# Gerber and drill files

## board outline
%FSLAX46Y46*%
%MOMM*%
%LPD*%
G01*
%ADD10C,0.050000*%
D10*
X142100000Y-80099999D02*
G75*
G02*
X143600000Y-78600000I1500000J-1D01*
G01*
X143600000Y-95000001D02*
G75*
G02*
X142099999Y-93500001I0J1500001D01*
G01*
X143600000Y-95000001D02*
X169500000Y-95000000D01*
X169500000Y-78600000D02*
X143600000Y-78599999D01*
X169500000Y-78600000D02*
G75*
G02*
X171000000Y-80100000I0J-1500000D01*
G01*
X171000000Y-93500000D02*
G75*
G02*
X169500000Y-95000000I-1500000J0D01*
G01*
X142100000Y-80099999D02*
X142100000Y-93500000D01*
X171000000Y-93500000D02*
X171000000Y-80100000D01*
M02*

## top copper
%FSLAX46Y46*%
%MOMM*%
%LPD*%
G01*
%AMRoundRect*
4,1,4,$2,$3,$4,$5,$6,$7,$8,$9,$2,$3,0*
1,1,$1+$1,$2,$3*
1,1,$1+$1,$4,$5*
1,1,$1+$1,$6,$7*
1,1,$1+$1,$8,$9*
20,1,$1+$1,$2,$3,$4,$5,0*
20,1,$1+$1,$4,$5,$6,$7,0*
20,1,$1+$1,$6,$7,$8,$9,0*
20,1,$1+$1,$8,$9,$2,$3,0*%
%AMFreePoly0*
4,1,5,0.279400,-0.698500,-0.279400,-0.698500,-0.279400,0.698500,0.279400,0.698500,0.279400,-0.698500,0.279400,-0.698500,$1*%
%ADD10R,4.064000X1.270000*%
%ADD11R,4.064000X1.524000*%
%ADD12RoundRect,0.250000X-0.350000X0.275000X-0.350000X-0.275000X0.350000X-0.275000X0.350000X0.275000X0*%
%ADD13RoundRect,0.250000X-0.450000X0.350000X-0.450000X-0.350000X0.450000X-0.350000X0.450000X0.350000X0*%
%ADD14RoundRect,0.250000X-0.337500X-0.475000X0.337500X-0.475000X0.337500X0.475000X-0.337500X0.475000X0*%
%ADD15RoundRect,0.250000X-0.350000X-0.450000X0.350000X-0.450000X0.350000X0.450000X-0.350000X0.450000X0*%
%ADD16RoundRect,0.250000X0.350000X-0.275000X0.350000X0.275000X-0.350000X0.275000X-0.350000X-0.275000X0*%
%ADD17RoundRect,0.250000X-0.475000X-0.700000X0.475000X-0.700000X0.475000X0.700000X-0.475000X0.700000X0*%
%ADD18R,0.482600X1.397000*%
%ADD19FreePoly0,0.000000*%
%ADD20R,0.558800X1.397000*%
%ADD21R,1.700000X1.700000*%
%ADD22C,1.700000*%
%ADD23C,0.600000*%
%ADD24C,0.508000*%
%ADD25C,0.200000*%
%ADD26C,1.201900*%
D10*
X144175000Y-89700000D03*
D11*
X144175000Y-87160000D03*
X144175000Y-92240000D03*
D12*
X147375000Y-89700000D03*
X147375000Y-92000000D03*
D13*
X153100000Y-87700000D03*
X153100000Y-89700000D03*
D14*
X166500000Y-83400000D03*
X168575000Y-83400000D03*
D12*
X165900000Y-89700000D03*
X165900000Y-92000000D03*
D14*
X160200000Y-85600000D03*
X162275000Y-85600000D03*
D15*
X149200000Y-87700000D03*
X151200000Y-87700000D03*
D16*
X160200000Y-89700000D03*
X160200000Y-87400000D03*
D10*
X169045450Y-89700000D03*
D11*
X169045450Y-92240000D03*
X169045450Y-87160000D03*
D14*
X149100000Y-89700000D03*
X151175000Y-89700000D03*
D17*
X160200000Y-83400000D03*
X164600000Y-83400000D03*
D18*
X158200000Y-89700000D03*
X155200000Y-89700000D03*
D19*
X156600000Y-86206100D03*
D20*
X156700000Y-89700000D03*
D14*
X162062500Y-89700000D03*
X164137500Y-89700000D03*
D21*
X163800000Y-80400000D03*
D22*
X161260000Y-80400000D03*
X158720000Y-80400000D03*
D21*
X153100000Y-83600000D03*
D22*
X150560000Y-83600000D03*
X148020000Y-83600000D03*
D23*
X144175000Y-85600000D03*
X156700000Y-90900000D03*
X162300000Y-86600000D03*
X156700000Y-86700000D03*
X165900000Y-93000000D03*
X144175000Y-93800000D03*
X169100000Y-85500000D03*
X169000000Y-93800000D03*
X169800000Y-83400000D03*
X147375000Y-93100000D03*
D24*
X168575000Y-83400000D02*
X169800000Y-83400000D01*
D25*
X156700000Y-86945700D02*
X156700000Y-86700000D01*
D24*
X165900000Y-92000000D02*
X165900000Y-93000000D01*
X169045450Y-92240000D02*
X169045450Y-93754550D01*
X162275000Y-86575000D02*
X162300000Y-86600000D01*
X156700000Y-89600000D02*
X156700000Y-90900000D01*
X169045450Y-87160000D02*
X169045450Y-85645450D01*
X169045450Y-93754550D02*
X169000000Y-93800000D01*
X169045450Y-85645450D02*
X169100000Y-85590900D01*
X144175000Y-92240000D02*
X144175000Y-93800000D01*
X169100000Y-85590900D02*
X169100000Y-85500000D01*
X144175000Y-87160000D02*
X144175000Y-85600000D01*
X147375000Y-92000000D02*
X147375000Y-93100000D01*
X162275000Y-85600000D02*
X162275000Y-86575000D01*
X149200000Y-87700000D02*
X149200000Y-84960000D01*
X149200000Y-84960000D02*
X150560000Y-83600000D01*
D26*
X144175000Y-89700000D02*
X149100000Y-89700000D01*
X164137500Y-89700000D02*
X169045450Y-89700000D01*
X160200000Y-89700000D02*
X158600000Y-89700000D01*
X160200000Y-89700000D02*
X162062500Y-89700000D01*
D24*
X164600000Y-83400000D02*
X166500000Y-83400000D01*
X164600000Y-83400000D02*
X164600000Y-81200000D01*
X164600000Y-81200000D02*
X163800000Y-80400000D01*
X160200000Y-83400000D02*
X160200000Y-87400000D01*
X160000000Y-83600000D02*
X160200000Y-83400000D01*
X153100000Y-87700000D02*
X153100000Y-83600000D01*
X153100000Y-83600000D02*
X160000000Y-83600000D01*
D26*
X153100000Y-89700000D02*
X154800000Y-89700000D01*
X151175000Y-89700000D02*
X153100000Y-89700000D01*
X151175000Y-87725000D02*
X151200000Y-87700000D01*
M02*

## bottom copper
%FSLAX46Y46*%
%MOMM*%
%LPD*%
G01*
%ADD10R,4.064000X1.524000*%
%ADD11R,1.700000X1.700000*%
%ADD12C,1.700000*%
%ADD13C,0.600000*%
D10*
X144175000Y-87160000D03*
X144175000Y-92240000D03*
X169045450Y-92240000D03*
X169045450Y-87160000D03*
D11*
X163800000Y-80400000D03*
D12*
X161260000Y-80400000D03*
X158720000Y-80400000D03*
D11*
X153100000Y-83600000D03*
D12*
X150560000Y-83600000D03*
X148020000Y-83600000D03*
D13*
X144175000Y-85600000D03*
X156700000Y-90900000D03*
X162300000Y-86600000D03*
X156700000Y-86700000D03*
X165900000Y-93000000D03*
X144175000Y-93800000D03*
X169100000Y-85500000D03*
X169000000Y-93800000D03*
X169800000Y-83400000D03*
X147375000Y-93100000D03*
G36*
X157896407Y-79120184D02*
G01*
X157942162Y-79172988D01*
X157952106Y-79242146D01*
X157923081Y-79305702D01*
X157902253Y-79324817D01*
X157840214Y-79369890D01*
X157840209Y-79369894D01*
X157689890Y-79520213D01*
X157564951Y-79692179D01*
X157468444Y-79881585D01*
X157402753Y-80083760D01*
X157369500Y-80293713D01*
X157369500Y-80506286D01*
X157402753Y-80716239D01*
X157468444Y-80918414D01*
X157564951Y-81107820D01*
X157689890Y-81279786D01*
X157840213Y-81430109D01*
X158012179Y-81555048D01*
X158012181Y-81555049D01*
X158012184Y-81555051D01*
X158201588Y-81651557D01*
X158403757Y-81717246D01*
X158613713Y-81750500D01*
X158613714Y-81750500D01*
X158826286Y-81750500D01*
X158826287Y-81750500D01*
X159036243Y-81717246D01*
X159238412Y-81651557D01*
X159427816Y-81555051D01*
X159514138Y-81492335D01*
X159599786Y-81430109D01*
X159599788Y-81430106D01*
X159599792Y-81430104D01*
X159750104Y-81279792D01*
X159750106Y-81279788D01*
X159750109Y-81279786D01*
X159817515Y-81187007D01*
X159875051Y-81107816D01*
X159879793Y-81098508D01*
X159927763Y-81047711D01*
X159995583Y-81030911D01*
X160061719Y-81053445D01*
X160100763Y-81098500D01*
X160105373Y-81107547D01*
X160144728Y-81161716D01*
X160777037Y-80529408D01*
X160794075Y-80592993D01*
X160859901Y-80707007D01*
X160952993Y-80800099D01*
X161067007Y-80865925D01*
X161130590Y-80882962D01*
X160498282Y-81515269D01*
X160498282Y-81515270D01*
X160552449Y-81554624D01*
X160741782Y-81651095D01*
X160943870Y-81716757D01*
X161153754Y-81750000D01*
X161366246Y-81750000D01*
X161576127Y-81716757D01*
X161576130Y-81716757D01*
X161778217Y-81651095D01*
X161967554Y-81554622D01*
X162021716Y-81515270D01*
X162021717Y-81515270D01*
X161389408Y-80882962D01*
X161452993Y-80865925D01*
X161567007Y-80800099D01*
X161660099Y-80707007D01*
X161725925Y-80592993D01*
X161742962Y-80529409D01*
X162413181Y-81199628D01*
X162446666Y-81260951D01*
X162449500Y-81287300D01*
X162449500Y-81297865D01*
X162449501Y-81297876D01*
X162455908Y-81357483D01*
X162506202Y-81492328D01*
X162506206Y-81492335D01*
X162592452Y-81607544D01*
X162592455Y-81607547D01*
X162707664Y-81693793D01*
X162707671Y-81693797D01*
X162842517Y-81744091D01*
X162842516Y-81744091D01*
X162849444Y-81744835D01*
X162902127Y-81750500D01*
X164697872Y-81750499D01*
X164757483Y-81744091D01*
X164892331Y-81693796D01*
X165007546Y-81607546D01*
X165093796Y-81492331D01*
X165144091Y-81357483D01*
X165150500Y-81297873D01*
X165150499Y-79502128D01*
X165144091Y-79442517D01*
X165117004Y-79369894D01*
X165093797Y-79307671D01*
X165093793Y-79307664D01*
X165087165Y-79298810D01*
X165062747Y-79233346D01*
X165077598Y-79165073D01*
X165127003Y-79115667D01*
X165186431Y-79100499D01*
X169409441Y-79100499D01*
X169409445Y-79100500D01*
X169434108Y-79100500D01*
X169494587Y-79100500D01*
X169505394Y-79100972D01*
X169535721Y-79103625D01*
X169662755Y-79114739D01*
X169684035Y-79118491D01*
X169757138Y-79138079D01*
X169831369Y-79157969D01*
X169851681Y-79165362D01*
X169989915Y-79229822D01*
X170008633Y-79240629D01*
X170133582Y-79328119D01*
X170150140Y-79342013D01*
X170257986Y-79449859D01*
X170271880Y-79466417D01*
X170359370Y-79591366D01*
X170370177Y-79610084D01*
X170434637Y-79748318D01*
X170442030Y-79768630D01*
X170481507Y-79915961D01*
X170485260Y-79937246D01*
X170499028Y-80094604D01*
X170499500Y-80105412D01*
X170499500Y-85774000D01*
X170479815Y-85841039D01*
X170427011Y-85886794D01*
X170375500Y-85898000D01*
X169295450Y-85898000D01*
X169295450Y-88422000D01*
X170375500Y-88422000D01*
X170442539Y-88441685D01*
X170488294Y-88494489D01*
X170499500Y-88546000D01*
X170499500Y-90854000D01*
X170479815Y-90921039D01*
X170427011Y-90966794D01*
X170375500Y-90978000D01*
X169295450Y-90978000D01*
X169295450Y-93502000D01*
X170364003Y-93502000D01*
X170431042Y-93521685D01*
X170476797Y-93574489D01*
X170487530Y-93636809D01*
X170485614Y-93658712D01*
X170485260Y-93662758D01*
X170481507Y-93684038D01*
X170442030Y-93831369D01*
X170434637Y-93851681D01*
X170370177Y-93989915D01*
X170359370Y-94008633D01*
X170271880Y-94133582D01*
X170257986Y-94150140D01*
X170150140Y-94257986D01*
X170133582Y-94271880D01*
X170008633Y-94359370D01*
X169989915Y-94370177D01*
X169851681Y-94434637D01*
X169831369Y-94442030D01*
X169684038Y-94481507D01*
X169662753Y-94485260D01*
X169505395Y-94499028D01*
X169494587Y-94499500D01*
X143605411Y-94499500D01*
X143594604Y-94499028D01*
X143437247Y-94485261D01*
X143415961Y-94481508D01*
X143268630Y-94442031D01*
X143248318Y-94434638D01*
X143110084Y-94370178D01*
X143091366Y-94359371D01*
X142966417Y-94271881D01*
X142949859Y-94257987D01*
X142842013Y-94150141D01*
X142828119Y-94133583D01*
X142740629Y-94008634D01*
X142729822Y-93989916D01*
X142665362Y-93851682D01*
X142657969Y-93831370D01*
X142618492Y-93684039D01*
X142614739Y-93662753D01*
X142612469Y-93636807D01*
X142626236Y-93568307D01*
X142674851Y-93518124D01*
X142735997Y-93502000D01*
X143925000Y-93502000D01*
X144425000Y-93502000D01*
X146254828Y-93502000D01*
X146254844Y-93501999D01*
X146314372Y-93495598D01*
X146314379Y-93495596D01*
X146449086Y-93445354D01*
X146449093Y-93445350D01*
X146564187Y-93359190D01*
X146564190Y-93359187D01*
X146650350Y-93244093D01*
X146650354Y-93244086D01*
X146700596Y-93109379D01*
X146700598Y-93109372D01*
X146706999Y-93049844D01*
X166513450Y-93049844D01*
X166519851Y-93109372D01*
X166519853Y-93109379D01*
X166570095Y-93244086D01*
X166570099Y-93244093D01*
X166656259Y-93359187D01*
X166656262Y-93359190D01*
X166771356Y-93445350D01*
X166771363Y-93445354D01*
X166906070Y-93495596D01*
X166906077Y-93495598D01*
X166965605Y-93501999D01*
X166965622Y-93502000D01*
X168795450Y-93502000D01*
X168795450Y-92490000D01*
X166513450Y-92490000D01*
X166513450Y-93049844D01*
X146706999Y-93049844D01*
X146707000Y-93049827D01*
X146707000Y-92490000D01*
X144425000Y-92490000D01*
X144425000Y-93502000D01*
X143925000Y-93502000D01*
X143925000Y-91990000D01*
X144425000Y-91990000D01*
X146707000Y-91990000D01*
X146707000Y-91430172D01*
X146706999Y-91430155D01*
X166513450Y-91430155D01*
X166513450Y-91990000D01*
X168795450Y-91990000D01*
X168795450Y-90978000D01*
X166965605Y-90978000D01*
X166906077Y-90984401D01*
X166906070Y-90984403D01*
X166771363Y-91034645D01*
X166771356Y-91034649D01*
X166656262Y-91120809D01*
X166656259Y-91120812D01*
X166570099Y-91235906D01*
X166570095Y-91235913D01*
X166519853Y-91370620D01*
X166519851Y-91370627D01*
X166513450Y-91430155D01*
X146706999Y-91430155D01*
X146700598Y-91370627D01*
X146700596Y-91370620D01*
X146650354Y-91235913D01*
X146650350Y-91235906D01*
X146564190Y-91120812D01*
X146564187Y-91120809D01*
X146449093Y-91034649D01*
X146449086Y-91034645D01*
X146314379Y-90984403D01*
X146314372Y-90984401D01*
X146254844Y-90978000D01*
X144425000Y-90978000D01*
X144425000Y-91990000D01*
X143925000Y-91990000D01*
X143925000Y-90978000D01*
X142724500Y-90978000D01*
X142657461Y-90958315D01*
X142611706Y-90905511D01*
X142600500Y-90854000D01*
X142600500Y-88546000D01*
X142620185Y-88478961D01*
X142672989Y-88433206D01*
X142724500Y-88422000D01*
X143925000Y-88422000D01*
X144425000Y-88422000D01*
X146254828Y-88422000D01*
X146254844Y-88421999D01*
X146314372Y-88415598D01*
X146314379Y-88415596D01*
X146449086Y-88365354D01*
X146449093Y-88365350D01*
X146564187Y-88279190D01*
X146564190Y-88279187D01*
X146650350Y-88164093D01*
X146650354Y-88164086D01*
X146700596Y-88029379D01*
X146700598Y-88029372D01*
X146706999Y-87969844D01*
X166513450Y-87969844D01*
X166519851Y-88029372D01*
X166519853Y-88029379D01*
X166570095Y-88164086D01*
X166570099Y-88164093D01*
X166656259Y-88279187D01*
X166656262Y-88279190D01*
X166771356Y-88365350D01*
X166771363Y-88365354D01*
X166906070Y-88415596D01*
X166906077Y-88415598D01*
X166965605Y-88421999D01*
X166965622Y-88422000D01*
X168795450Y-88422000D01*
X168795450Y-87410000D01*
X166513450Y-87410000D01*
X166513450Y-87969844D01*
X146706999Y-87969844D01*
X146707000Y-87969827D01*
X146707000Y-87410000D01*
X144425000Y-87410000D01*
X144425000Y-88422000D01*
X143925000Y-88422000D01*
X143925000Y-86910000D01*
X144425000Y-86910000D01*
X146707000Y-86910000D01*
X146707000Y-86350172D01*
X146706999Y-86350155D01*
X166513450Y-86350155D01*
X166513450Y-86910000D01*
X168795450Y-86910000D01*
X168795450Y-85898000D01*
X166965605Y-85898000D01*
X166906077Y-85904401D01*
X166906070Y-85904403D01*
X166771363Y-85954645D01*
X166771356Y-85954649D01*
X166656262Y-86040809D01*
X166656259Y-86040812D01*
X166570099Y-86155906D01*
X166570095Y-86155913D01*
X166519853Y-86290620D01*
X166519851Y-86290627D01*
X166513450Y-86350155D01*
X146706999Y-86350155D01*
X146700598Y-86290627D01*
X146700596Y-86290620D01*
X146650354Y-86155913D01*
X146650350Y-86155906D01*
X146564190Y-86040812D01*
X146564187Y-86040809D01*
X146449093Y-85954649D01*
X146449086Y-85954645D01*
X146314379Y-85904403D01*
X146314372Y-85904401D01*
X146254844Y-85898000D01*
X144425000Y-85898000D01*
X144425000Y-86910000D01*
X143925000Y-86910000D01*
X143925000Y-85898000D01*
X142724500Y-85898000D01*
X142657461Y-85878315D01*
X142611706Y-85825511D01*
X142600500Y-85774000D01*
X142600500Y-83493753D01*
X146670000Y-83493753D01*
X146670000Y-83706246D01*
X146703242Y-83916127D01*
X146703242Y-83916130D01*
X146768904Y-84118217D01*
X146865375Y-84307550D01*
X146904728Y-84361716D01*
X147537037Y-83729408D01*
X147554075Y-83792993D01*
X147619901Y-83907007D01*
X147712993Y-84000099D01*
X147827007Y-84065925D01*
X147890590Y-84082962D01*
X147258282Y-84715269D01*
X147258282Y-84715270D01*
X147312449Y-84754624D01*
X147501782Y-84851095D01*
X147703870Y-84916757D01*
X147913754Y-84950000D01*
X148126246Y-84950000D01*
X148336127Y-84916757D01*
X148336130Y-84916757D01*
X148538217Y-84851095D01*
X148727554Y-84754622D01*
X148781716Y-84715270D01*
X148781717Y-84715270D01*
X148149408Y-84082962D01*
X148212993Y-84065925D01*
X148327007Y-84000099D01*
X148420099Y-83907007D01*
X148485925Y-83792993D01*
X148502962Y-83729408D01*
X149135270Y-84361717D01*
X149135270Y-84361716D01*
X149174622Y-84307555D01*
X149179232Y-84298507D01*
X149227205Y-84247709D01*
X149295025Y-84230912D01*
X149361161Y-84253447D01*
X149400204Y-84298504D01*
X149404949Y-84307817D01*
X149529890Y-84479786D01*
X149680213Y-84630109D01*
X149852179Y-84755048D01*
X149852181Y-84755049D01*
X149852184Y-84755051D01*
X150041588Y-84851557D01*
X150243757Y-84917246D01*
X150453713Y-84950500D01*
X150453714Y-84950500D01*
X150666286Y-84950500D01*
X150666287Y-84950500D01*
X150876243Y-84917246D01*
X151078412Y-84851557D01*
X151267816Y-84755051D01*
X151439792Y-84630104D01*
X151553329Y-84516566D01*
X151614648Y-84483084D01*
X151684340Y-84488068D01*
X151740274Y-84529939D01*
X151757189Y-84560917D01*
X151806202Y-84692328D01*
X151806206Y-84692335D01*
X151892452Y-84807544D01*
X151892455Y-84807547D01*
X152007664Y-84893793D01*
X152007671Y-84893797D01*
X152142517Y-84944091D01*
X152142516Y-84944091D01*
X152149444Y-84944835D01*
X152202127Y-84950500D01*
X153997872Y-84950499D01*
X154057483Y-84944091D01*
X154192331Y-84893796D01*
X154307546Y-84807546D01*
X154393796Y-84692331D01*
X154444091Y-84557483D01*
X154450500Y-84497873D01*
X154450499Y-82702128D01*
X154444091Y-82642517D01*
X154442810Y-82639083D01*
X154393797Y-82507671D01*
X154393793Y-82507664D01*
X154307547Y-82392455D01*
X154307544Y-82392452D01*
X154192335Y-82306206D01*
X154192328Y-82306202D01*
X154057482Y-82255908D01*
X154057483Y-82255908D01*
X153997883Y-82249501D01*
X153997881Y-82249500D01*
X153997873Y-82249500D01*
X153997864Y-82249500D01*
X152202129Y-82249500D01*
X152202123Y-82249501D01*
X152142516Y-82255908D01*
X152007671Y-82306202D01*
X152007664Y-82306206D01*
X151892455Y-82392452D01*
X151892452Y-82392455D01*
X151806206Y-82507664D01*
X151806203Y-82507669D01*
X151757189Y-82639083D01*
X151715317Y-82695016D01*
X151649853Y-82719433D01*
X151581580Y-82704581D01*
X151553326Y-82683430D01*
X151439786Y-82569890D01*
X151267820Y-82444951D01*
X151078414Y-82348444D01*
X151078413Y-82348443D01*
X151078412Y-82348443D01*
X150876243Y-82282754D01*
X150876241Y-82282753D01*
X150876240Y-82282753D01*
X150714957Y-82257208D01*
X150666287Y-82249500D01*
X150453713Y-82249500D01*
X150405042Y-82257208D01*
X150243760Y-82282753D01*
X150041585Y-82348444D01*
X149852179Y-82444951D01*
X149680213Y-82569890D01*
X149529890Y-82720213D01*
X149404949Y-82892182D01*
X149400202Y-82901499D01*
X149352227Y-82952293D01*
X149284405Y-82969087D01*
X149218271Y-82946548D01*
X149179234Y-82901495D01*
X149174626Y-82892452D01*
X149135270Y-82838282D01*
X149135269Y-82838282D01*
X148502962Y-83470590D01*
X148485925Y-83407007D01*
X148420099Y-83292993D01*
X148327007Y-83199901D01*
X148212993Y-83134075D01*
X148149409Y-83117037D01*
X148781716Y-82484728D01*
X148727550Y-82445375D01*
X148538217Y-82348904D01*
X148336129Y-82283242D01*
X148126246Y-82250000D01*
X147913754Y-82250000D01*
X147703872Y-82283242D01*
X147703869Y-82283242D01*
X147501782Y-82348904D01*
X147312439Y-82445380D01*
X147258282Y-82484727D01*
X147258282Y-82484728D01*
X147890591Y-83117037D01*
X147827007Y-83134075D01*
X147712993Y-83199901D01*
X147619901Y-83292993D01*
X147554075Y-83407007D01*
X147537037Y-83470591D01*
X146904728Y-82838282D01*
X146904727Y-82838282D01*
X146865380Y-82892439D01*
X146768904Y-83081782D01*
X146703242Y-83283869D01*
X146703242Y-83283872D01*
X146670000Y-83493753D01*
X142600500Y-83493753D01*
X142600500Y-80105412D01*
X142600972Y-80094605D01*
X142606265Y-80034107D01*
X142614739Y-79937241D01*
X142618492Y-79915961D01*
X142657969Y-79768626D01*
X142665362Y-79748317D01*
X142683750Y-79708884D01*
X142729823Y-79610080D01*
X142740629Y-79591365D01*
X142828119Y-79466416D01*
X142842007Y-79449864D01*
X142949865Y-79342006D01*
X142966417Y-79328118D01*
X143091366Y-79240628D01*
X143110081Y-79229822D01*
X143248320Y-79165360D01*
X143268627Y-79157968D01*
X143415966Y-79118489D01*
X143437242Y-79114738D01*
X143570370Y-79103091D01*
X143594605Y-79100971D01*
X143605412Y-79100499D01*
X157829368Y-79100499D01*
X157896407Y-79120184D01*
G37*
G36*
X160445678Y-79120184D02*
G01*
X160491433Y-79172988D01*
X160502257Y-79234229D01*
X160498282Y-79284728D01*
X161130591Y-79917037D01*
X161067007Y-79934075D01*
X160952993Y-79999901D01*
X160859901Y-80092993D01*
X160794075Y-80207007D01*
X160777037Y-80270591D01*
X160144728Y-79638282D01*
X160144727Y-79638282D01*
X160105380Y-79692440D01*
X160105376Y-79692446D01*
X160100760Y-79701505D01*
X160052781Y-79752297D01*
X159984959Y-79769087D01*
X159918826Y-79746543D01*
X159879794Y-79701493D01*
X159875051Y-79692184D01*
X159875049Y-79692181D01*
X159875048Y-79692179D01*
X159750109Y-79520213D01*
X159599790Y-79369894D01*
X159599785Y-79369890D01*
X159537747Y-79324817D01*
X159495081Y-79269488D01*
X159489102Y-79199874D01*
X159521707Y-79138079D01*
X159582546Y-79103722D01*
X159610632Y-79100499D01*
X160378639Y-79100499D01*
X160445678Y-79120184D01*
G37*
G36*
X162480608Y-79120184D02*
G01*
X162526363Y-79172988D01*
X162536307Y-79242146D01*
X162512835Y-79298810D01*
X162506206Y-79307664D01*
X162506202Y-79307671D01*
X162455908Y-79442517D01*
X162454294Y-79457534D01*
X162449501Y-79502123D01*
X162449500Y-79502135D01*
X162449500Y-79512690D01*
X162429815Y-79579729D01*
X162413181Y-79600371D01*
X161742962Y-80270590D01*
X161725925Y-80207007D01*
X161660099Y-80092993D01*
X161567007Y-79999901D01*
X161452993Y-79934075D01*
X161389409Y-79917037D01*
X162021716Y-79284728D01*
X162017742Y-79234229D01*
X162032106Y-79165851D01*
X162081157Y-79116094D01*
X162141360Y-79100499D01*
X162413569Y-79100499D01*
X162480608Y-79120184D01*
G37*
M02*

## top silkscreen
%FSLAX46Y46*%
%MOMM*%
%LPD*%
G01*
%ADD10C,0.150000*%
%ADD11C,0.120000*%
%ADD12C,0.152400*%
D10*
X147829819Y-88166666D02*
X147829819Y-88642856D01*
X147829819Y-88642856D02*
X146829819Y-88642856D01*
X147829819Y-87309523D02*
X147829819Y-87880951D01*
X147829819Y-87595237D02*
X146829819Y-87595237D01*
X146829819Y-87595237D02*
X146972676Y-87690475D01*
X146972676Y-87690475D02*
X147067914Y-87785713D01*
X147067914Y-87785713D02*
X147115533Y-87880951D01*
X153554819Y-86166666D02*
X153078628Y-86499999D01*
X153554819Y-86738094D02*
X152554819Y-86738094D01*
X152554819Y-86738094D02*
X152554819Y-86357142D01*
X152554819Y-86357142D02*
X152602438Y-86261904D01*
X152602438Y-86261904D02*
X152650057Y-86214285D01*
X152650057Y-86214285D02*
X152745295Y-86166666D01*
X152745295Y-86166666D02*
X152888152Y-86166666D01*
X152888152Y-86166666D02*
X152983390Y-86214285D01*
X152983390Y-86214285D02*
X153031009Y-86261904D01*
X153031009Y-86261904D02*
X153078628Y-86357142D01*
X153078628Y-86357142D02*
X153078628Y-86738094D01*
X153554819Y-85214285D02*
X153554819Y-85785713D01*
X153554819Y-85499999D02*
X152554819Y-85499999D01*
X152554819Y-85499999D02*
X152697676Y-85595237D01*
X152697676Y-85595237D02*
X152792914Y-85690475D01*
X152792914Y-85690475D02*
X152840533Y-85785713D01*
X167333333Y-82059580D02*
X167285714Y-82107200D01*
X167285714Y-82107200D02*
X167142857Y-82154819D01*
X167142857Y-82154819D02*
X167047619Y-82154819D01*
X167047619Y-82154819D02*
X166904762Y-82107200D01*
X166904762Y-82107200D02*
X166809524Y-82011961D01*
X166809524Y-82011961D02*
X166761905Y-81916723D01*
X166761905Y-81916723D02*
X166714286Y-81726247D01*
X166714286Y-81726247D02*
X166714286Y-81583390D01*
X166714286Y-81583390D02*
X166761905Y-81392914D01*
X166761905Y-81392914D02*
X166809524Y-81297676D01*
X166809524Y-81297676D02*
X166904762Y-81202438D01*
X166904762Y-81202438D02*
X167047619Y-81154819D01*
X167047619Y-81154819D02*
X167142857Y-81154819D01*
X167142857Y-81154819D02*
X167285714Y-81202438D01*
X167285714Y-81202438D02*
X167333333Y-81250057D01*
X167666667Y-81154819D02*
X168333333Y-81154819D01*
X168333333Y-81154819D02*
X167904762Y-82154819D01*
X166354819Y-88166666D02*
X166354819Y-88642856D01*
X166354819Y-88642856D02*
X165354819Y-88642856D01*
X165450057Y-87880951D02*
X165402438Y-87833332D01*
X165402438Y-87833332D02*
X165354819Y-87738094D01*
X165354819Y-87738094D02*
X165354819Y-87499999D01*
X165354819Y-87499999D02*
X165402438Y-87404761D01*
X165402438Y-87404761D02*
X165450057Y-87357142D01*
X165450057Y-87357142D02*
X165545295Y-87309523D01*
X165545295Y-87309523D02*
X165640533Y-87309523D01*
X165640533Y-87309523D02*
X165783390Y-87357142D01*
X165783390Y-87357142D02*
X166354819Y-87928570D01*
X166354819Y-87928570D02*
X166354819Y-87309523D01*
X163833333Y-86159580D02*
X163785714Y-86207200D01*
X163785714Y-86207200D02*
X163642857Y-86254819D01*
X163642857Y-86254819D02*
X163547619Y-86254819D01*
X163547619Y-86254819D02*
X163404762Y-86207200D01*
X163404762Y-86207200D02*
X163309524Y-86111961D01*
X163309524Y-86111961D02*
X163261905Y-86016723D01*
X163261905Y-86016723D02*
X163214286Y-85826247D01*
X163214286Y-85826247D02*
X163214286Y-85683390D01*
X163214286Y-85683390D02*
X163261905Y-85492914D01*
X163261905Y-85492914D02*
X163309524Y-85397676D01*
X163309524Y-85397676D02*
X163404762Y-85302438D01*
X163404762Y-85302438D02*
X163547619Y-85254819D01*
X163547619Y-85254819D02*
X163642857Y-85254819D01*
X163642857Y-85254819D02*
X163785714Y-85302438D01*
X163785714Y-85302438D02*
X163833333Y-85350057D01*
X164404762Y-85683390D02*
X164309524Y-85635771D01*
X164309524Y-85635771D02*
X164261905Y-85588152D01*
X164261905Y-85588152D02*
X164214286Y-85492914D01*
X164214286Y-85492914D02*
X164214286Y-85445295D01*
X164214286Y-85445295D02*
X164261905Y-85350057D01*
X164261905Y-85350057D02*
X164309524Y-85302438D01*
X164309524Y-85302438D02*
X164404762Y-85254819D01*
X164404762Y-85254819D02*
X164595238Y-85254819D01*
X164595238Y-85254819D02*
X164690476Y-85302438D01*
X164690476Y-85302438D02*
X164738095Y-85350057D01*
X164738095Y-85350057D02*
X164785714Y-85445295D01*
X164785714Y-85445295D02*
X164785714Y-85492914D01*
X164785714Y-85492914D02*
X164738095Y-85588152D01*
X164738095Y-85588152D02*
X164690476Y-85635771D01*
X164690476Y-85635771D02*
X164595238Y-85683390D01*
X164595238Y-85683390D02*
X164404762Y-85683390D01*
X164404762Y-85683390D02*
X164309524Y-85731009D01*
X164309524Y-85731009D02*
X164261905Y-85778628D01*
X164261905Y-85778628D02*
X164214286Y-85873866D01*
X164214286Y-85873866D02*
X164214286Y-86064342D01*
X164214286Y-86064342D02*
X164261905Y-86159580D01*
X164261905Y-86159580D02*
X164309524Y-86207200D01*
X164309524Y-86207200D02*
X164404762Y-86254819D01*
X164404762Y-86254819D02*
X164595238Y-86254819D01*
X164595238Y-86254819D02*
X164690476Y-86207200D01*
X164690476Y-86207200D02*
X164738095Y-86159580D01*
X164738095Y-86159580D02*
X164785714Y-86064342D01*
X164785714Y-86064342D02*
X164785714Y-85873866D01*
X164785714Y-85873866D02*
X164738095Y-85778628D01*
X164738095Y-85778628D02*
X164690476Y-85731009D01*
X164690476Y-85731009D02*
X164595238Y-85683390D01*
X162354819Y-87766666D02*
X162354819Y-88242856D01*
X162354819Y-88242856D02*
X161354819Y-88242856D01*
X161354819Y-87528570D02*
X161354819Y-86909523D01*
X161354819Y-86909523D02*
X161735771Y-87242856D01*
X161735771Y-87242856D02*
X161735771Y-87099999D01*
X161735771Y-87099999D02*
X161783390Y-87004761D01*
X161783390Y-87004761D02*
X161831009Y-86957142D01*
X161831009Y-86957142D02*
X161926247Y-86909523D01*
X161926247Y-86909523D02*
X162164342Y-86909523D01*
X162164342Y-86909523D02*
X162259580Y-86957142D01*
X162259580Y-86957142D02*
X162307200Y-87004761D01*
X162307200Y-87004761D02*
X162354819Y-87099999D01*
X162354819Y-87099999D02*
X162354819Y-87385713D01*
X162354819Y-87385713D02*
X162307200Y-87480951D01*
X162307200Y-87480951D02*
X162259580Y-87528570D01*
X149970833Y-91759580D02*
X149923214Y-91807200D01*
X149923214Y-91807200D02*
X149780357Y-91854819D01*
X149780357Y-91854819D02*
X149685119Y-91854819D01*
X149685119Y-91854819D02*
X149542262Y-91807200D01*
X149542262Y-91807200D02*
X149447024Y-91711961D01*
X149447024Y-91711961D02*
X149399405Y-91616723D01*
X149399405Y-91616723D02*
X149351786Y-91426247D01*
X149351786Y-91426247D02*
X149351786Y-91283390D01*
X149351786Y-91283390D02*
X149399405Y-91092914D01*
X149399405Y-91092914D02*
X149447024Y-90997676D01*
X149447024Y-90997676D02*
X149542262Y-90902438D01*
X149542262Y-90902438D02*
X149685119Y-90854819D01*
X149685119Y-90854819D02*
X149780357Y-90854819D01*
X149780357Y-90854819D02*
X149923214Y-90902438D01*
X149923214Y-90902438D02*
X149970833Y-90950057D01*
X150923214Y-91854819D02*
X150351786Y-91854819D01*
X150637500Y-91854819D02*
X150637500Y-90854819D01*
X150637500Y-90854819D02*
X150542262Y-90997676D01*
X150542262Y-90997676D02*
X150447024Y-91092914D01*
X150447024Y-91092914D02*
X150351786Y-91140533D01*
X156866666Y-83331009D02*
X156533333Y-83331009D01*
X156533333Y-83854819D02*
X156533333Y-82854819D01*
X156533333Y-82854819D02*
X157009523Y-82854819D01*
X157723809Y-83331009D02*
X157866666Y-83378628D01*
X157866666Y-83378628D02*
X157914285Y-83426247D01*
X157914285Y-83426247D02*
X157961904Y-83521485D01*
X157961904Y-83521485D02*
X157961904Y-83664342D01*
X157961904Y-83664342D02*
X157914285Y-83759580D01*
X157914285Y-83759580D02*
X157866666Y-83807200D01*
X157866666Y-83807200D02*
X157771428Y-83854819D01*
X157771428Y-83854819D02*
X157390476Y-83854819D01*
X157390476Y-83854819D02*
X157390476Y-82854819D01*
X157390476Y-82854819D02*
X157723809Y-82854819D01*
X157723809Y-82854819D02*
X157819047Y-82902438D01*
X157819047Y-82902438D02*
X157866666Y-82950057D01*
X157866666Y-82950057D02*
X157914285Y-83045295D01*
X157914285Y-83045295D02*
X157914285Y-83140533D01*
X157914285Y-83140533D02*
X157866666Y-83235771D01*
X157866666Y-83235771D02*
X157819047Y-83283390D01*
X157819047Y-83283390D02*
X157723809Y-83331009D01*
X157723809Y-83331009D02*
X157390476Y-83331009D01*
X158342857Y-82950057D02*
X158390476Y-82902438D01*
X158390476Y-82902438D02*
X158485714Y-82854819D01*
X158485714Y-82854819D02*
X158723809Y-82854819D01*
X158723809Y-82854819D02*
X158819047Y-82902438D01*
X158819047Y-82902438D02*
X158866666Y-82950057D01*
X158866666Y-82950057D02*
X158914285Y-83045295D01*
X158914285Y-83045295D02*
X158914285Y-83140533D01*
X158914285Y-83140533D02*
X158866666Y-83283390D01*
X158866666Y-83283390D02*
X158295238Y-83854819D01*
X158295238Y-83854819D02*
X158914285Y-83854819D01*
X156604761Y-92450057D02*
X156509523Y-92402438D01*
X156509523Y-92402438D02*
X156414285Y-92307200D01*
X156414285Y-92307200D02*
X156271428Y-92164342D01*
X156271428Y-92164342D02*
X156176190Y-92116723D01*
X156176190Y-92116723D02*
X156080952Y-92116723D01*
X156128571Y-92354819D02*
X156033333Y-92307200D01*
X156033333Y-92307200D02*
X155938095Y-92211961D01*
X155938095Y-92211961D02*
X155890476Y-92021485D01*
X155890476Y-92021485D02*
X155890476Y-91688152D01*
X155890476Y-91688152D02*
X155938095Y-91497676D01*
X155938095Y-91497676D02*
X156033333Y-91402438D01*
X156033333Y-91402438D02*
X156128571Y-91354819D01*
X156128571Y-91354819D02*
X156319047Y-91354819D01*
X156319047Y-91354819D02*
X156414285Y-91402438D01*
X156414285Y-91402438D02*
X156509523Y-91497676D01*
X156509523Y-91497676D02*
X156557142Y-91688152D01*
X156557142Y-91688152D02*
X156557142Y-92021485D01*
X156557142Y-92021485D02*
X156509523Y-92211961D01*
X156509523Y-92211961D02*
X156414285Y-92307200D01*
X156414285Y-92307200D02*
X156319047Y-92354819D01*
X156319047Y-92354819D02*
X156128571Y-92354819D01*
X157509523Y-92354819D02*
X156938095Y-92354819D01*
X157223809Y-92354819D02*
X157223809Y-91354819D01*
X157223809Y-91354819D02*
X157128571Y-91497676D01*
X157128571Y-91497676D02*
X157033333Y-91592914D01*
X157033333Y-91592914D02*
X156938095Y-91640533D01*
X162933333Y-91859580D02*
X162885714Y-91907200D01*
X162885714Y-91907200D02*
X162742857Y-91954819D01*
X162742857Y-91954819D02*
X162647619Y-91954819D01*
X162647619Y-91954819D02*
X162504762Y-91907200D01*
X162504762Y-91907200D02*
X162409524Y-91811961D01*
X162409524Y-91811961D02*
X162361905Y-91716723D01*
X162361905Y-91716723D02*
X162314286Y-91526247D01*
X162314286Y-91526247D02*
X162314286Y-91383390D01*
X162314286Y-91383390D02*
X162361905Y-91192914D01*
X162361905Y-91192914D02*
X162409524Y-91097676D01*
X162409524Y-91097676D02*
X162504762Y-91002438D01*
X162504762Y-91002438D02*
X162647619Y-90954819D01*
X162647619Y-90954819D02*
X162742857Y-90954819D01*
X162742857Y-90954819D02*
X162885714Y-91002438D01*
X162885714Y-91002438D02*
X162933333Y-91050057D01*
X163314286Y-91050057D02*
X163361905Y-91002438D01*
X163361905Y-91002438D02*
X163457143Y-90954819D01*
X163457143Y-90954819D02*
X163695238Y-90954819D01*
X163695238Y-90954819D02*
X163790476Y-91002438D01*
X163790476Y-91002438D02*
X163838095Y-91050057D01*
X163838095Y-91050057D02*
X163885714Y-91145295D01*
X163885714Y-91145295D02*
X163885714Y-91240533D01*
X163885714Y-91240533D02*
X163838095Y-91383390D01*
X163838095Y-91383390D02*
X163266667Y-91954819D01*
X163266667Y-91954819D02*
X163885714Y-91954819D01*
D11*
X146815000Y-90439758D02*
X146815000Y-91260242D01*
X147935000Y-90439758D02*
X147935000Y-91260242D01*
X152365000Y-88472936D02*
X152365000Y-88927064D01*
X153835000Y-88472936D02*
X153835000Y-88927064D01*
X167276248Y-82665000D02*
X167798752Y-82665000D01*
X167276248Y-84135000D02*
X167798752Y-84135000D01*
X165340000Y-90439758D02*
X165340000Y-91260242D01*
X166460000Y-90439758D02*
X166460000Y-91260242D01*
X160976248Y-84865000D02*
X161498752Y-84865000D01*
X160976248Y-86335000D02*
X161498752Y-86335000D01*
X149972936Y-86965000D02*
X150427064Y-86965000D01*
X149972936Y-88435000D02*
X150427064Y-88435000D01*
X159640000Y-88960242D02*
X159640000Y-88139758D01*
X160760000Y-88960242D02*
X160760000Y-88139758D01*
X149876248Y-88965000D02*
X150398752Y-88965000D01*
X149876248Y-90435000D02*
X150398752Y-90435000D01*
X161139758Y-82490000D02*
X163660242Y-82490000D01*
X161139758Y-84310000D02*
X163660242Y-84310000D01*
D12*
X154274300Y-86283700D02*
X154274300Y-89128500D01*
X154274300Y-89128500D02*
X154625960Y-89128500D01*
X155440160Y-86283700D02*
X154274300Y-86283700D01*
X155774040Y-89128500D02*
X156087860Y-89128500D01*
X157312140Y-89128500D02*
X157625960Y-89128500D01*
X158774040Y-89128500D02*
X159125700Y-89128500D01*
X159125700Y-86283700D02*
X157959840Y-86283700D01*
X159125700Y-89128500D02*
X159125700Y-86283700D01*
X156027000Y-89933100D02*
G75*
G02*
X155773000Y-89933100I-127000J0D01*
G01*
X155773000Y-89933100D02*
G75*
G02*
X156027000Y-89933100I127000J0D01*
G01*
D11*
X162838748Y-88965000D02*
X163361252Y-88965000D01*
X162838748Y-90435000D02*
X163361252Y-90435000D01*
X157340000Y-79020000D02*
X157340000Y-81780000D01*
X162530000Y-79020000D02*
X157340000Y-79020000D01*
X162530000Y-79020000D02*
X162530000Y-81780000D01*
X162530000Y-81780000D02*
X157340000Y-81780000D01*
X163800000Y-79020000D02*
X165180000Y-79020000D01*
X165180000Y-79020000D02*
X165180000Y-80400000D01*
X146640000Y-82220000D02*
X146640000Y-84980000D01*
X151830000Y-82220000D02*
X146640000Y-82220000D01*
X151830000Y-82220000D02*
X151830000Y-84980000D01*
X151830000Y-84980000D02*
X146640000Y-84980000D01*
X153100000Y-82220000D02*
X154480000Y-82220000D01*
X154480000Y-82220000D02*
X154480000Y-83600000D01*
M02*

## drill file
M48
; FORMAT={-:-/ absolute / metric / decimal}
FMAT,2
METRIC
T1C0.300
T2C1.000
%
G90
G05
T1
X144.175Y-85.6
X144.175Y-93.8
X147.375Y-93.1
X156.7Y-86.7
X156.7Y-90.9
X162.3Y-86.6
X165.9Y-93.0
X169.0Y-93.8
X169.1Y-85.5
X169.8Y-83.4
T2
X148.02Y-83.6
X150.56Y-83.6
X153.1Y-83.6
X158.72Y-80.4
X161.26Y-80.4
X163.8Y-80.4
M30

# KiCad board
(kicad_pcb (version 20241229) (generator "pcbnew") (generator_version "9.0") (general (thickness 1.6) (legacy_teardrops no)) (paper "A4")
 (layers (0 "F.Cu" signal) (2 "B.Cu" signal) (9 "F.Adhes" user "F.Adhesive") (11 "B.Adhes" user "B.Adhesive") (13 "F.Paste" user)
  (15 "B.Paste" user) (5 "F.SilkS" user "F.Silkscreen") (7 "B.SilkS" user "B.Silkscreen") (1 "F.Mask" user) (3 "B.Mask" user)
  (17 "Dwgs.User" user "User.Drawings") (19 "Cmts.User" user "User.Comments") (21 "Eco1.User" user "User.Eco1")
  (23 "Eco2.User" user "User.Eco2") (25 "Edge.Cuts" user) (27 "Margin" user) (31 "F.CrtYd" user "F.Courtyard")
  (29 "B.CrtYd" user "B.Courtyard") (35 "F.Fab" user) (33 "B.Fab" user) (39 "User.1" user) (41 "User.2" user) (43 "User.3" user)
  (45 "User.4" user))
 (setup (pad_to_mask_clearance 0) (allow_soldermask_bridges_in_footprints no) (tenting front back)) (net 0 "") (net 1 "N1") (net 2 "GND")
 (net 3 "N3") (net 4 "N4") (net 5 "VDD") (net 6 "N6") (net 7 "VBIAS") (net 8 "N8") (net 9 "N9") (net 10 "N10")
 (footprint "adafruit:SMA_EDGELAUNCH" (layer "F.Cu") (at 142.143 89.7)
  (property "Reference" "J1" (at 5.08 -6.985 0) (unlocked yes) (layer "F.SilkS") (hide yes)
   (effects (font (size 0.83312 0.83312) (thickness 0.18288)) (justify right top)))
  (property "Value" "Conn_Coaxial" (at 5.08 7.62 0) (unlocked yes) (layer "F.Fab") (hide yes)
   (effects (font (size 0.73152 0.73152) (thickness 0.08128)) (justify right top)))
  (pad "1" smd rect (at 2.032 0 90) (size 1.27 4.064) (layers "F.Cu" "F.Mask") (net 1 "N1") (solder_mask_margin 0.1016) (zone_connect 2)
   (thermal_bridge_angle 0))
  (pad "2" smd rect (at 2.032 -2.54 90) (size 1.524 4.064) (layers "F.Cu" "F.Mask") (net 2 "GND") (solder_mask_margin 0.1016)
   (thermal_bridge_angle 0))
  (pad "2" smd rect (at 2.032 -2.54 90) (size 1.524 4.064) (layers "B.Cu" "B.Mask") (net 2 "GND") (solder_mask_margin 0.1016)
   (thermal_bridge_angle 0))
  (pad "2" smd rect (at 2.032 2.54 90) (size 1.524 4.064) (layers "F.Cu" "F.Mask") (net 2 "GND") (solder_mask_margin 0.1016)
   (thermal_bridge_angle 0))
  (pad "2" smd rect (at 2.032 2.54 90) (size 1.524 4.064) (layers "B.Cu" "B.Mask") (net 2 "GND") (solder_mask_margin 0.1016)
   (thermal_bridge_angle 0)))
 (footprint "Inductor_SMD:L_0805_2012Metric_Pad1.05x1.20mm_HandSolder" (layer "F.Cu") (at 147.375 90.85 -90)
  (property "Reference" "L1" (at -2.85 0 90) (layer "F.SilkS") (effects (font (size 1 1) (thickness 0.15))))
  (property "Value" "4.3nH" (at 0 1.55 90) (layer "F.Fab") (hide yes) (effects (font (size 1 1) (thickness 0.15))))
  (fp_line (start -0.410242 0.56) (end 0.410242 0.56) (stroke (width 0.12) (type solid)) (layer "F.SilkS"))
  (fp_line (start -0.410242 -0.56) (end 0.410242 -0.56) (stroke (width 0.12) (type solid)) (layer "F.SilkS"))
  (pad "1" smd roundrect (at -1.15 0 270) (size 1.05 1.2) (layers "F.Cu" "F.Mask" "F.Paste") (roundrect_rratio 0.238095) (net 1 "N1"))
  (pad "2" smd roundrect (at 1.15 0 270) (size 1.05 1.2) (layers "F.Cu" "F.Mask" "F.Paste") (roundrect_rratio 0.238095) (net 2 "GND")))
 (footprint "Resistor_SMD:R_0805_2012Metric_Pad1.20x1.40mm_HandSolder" (layer "F.Cu") (at 153.1 88.7 -90)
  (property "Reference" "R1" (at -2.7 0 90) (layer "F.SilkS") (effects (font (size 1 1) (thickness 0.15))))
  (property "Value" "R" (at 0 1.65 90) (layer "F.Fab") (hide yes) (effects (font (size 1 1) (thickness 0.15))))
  (fp_line (start -0.227064 0.735) (end 0.227064 0.735) (stroke (width 0.12) (type solid)) (layer "F.SilkS"))
  (fp_line (start -0.227064 -0.735) (end 0.227064 -0.735) (stroke (width 0.12) (type solid)) (layer "F.SilkS"))
  (pad "1" smd roundrect (at -1 0 270) (size 1.2 1.4) (layers "F.Cu" "F.Mask" "F.Paste") (roundrect_rratio 0.208333) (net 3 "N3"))
  (pad "2" smd roundrect (at 1 0 270) (size 1.2 1.4) (layers "F.Cu" "F.Mask" "F.Paste") (roundrect_rratio 0.208333) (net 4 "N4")))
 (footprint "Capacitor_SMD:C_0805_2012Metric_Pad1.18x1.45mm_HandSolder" (layer "F.Cu") (at 167.5375 83.4)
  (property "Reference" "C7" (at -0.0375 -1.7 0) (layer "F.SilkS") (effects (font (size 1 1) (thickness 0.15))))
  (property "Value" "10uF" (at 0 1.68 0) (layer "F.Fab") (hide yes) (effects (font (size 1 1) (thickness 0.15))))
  (fp_line (start -0.261252 -0.735) (end 0.261252 -0.735) (stroke (width 0.12) (type solid)) (layer "F.SilkS"))
  (fp_line (start -0.261252 0.735) (end 0.261252 0.735) (stroke (width 0.12) (type solid)) (layer "F.SilkS"))
  (pad "1" smd roundrect (at -1.0375 0) (size 1.175 1.45) (layers "F.Cu" "F.Mask" "F.Paste") (roundrect_rratio 0.212766) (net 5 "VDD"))
  (pad "2" smd roundrect (at 1.0375 0) (size 1.175 1.45) (layers "F.Cu" "F.Mask" "F.Paste") (roundrect_rratio 0.212766) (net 2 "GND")))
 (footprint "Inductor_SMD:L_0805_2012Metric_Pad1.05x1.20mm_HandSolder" (layer "F.Cu") (at 165.9 90.85 -90)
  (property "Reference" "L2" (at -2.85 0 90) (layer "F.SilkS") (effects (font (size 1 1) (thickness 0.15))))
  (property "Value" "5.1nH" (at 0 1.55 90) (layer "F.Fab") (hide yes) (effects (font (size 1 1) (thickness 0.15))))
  (fp_line (start -0.410242 0.56) (end 0.410242 0.56) (stroke (width 0.12) (type solid)) (layer "F.SilkS"))
  (fp_line (start -0.410242 -0.56) (end 0.410242 -0.56) (stroke (width 0.12) (type solid)) (layer "F.SilkS"))
  (pad "1" smd roundrect (at -1.15 0 270) (size 1.05 1.2) (layers "F.Cu" "F.Mask" "F.Paste") (roundrect_rratio 0.238095) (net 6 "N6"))
  (pad "2" smd roundrect (at 1.15 0 270) (size 1.05 1.2) (layers "F.Cu" "F.Mask" "F.Paste") (roundrect_rratio 0.238095) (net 2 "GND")))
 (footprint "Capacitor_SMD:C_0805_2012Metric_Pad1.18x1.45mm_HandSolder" (layer "F.Cu") (at 161.2375 85.6)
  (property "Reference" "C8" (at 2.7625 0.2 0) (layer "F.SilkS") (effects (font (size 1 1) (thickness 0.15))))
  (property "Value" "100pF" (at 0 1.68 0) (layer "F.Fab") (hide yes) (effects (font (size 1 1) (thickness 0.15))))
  (fp_line (start -0.261252 -0.735) (end 0.261252 -0.735) (stroke (width 0.12) (type solid)) (layer "F.SilkS"))
  (fp_line (start -0.261252 0.735) (end 0.261252 0.735) (stroke (width 0.12) (type solid)) (layer "F.SilkS"))
  (pad "1" smd roundrect (at -1.0375 0) (size 1.175 1.45) (layers "F.Cu" "F.Mask" "F.Paste") (roundrect_rratio 0.212766) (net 3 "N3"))
  (pad "2" smd roundrect (at 1.0375 0) (size 1.175 1.45) (layers "F.Cu" "F.Mask" "F.Paste") (roundrect_rratio 0.212766) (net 2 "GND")))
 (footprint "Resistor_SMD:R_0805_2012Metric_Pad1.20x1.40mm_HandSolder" (layer "F.Cu") (at 150.2 87.7)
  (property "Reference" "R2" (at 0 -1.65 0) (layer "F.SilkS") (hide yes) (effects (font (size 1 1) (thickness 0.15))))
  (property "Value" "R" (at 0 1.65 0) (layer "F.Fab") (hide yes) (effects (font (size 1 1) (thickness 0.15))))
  (fp_line (start -0.227064 -0.735) (end 0.227064 -0.735) (stroke (width 0.12) (type solid)) (layer "F.SilkS"))
  (fp_line (start -0.227064 0.735) (end 0.227064 0.735) (stroke (width 0.12) (type solid)) (layer "F.SilkS"))
  (pad "1" smd roundrect (at -1 0) (size 1.2 1.4) (layers "F.Cu" "F.Mask" "F.Paste") (roundrect_rratio 0.208333) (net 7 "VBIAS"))
  (pad "2" smd roundrect (at 1 0) (size 1.2 1.4) (layers "F.Cu" "F.Mask" "F.Paste") (roundrect_rratio 0.208333) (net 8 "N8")))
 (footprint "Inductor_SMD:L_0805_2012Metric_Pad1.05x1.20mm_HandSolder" (layer "F.Cu") (at 160.2 88.55 90)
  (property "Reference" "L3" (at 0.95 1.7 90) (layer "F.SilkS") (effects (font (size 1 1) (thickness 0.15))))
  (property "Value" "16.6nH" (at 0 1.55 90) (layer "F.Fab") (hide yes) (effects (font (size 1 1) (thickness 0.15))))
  (fp_line (start -0.410242 -0.56) (end 0.410242 -0.56) (stroke (width 0.12) (type solid)) (layer "F.SilkS"))
  (fp_line (start -0.410242 0.56) (end 0.410242 0.56) (stroke (width 0.12) (type solid)) (layer "F.SilkS"))
  (pad "1" smd roundrect (at -1.15 0 90) (size 1.05 1.2) (layers "F.Cu" "F.Mask" "F.Paste") (roundrect_rratio 0.238095) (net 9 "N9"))
  (pad "2" smd roundrect (at 1.15 0 90) (size 1.05 1.2) (layers "F.Cu" "F.Mask" "F.Paste") (roundrect_rratio 0.238095) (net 3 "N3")))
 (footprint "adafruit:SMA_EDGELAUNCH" (layer "F.Cu") (at 171.07745 89.7 180)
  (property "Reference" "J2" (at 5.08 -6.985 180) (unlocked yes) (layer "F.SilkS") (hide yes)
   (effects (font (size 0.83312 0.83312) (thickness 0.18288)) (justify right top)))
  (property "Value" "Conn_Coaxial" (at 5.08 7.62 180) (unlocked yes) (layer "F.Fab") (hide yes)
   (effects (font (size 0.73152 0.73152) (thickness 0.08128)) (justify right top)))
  (pad "1" smd rect (at 2.032 0 270) (size 1.27 4.064) (layers "F.Cu" "F.Mask") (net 6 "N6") (solder_mask_margin 0.1016) (zone_connect 2)
   (thermal_bridge_angle 0))
  (pad "2" smd rect (at 2.032 -2.54 270) (size 1.524 4.064) (layers "F.Cu" "F.Mask") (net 2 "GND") (solder_mask_margin 0.1016)
   (thermal_bridge_angle 0))
  (pad "2" smd rect (at 2.032 -2.54 270) (size 1.524 4.064) (layers "B.Cu" "B.Mask") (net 2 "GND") (solder_mask_margin 0.1016)
   (thermal_bridge_angle 0))
  (pad "2" smd rect (at 2.032 2.54 270) (size 1.524 4.064) (layers "F.Cu" "F.Mask") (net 2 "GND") (solder_mask_margin 0.1016)
   (thermal_bridge_angle 0))
  (pad "2" smd rect (at 2.032 2.54 270) (size 1.524 4.064) (layers "B.Cu" "B.Mask") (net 2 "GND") (solder_mask_margin 0.1016)
   (thermal_bridge_angle 0)))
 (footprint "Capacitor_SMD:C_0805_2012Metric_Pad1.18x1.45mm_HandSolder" (layer "F.Cu") (at 150.1375 89.7)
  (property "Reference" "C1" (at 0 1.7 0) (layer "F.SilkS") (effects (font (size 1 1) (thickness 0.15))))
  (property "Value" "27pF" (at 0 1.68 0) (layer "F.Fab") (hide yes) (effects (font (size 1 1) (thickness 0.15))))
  (fp_line (start -0.261252 -0.735) (end 0.261252 -0.735) (stroke (width 0.12) (type solid)) (layer "F.SilkS"))
  (fp_line (start -0.261252 0.735) (end 0.261252 0.735) (stroke (width 0.12) (type solid)) (layer "F.SilkS"))
  (pad "1" smd roundrect (at -1.0375 0) (size 1.175 1.45) (layers "F.Cu" "F.Mask" "F.Paste") (roundrect_rratio 0.212766) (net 1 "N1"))
  (pad "2" smd roundrect (at 1.0375 0) (size 1.175 1.45) (layers "F.Cu" "F.Mask" "F.Paste") (roundrect_rratio 0.212766) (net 4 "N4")))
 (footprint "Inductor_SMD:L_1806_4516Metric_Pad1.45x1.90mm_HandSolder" (layer "F.Cu") (at 162.4 83.4)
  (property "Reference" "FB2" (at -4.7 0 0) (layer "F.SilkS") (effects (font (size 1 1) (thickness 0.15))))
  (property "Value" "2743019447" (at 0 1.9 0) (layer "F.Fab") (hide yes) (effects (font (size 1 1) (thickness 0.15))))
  (fp_line (start -1.260242 -0.91) (end 1.260242 -0.91) (stroke (width 0.12) (type solid)) (layer "F.SilkS"))
  (fp_line (start -1.260242 0.91) (end 1.260242 0.91) (stroke (width 0.12) (type solid)) (layer "F.SilkS"))
  (pad "1" smd roundrect (at -2.2 0) (size 1.45 1.9) (layers "F.Cu" "F.Mask" "F.Paste") (roundrect_rratio 0.172414) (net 3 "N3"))
  (pad "2" smd roundrect (at 2.2 0) (size 1.45 1.9) (layers "F.Cu" "F.Mask" "F.Paste") (roundrect_rratio 0.172414) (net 5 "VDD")))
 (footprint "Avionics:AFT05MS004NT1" (layer "F.Cu") (at 156.7 87.7061)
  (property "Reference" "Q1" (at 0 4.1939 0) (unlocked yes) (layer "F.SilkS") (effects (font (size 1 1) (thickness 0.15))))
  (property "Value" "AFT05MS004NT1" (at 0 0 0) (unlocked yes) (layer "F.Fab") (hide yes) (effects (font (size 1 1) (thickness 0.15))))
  (fp_line (start -2.4257 -1.4224) (end -2.4257 1.4224) (stroke (width 0.1524) (type solid)) (layer "F.SilkS"))
  (fp_line (start -2.4257 1.4224) (end -2.07404 1.4224) (stroke (width 0.1524) (type solid)) (layer "F.SilkS"))
  (fp_line (start -1.25984 -1.4224) (end -2.4257 -1.4224) (stroke (width 0.1524) (type solid)) (layer "F.SilkS"))
  (fp_line (start -0.92596 1.4224) (end -0.61214 1.4224) (stroke (width 0.1524) (type solid)) (layer "F.SilkS"))
  (fp_line (start 0.61214 1.4224) (end 0.92596 1.4224) (stroke (width 0.1524) (type solid)) (layer "F.SilkS"))
  (fp_line (start 2.07404 1.4224) (end 2.4257 1.4224) (stroke (width 0.1524) (type solid)) (layer "F.SilkS"))
  (fp_line (start 2.4257 -1.4224) (end 1.25984 -1.4224) (stroke (width 0.1524) (type solid)) (layer "F.SilkS"))
  (fp_line (start 2.4257 1.4224) (end 2.4257 -1.4224) (stroke (width 0.1524) (type solid)) (layer "F.SilkS"))
  (fp_circle (center -0.8 2.227) (end -0.673 2.227) (stroke (width 0.1524) (type solid)) (fill no) (layer "F.SilkS"))
  (pad "1" smd rect (at 1.5 1.9939) (size 0.4826 1.397) (layers "F.Cu" "F.Mask" "F.Paste") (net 9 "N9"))
  (pad "2" smd rect (at -1.5 1.9939) (size 0.4826 1.397) (layers "F.Cu" "F.Mask" "F.Paste") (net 4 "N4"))
  (pad "3" smd custom (at -0.1 -1.5) (size 0.5588 1.397) (layers "F.Cu" "F.Mask" "F.Paste") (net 2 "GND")
   (options (clearance outline) (anchor rect)) (primitives))
  (pad "3" smd rect (at 0 1.9939) (size 0.5588 1.397) (layers "F.Cu" "F.Mask" "F.Paste") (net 2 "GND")))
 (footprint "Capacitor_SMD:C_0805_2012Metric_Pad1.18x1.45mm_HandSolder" (layer "F.Cu") (at 163.1 89.7)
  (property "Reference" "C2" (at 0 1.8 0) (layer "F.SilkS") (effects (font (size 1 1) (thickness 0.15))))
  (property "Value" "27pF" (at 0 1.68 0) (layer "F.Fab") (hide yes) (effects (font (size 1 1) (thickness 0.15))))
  (fp_line (start -0.261252 -0.735) (end 0.261252 -0.735) (stroke (width 0.12) (type solid)) (layer "F.SilkS"))
  (fp_line (start -0.261252 0.735) (end 0.261252 0.735) (stroke (width 0.12) (type solid)) (layer "F.SilkS"))
  (pad "1" smd roundrect (at -1.0375 0) (size 1.175 1.45) (layers "F.Cu" "F.Mask" "F.Paste") (roundrect_rratio 0.212766) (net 9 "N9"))
  (pad "2" smd roundrect (at 1.0375 0) (size 1.175 1.45) (layers "F.Cu" "F.Mask" "F.Paste") (roundrect_rratio 0.212766) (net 6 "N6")))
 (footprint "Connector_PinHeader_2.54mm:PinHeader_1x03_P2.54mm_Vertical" (layer "F.Cu") (at 163.8 80.4 -90)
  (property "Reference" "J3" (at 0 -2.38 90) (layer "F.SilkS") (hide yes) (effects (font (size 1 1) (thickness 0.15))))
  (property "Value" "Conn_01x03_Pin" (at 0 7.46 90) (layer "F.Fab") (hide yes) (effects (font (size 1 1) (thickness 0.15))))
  (fp_line (start -1.38 6.46) (end 1.38 6.46) (stroke (width 0.12) (type solid)) (layer "F.SilkS"))
  (fp_line (start -1.38 1.27) (end -1.38 6.46) (stroke (width 0.12) (type solid)) (layer "F.SilkS"))
  (fp_line (start -1.38 1.27) (end 1.38 1.27) (stroke (width 0.12) (type solid)) (layer "F.SilkS"))
  (fp_line (start 1.38 1.27) (end 1.38 6.46) (stroke (width 0.12) (type solid)) (layer "F.SilkS"))
  (fp_line (start -1.38 0) (end -1.38 -1.38) (stroke (width 0.12) (type solid)) (layer "F.SilkS"))
  (fp_line (start -1.38 -1.38) (end 0 -1.38) (stroke (width 0.12) (type solid)) (layer "F.SilkS"))
  (pad "1" thru_hole rect (at 0 0 270) (size 1.7 1.7) (drill 1) (layers "*.Cu" "*.Mask") (remove_unused_layers no) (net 5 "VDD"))
  (pad "2" thru_hole circle (at 0 2.54 270) (size 1.7 1.7) (drill 1) (layers "*.Cu" "*.Mask") (remove_unused_layers no) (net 2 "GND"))
  (pad "3" thru_hole circle (at 0 5.08 270) (size 1.7 1.7) (drill 1) (layers "*.Cu" "*.Mask") (remove_unused_layers no) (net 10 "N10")))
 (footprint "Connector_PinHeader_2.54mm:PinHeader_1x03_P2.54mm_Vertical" (layer "F.Cu") (at 153.1 83.6 -90)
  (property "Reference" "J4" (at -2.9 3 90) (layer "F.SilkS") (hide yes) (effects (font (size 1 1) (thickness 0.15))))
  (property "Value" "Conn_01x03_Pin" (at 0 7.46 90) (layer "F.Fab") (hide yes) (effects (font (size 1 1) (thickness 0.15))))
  (fp_line (start -1.38 6.46) (end 1.38 6.46) (stroke (width 0.12) (type solid)) (layer "F.SilkS"))
  (fp_line (start -1.38 1.27) (end -1.38 6.46) (stroke (width 0.12) (type solid)) (layer "F.SilkS"))
  (fp_line (start -1.38 1.27) (end 1.38 1.27) (stroke (width 0.12) (type solid)) (layer "F.SilkS"))
  (fp_line (start 1.38 1.27) (end 1.38 6.46) (stroke (width 0.12) (type solid)) (layer "F.SilkS"))
  (fp_line (start -1.38 0) (end -1.38 -1.38) (stroke (width 0.12) (type solid)) (layer "F.SilkS"))
  (fp_line (start -1.38 -1.38) (end 0 -1.38) (stroke (width 0.12) (type solid)) (layer "F.SilkS"))
  (pad "1" thru_hole rect (at 0 0 270) (size 1.7 1.7) (drill 1) (layers "*.Cu" "*.Mask") (remove_unused_layers no) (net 3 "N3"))
  (pad "2" thru_hole circle (at 0 2.54 270) (size 1.7 1.7) (drill 1) (layers "*.Cu" "*.Mask") (remove_unused_layers no) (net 7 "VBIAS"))
  (pad "3" thru_hole circle (at 0 5.08 270) (size 1.7 1.7) (drill 1) (layers "*.Cu" "*.Mask") (remove_unused_layers no) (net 2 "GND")))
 (gr_arc (start 142.1 80.099999) (mid 142.53934 79.039339) (end 143.6 78.599999) (stroke (width 0.05) (type default)) (layer "Edge.Cuts"))
 (gr_arc (start 143.6 95.000001) (mid 142.53934 94.560661) (end 142.1 93.500001) (stroke (width 0.05) (type default)) (layer "Edge.Cuts"))
 (gr_line (start 143.6 95.000001) (end 169.5 95) (stroke (width 0.05) (type default)) (layer "Edge.Cuts"))
 (gr_line (start 169.5 78.6) (end 143.6 78.599999) (stroke (width 0.05) (type default)) (layer "Edge.Cuts"))
 (gr_arc (start 169.5 78.6) (mid 170.56066 79.03934) (end 171 80.1) (stroke (width 0.05) (type default)) (layer "Edge.Cuts"))
 (gr_arc (start 171 93.5) (mid 170.56066 94.56066) (end 169.5 95) (stroke (width 0.05) (type default)) (layer "Edge.Cuts"))
 (gr_line (start 142.1 80.099999) (end 142.1 93.5) (stroke (width 0.05) (type default)) (layer "Edge.Cuts"))
 (gr_line (start 171 93.5) (end 171 80.1) (stroke (width 0.05) (type default)) (layer "Edge.Cuts"))
 (segment (start 168.575 83.4) (end 169.8 83.4) (width 0.508) (layer "F.Cu") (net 2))
 (segment (start 156.7 86.9457) (end 156.7 86.7) (width 0.2) (layer "F.Cu") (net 2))
 (segment (start 165.9 92) (end 165.9 93) (width 0.508) (layer "F.Cu") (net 2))
 (segment (start 169.04545 92.24) (end 169.04545 93.75455) (width 0.508) (layer "F.Cu") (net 2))
 (segment (start 162.275 86.575) (end 162.3 86.6) (width 0.508) (layer "F.Cu") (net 2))
 (segment (start 156.7 89.6) (end 156.7 90.9) (width 0.508) (layer "F.Cu") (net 2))
 (segment (start 169.04545 87.16) (end 169.04545 85.64545) (width 0.508) (layer "F.Cu") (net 2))
 (segment (start 169.04545 93.75455) (end 169 93.8) (width 0.508) (layer "F.Cu") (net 2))
 (segment (start 169.04545 85.64545) (end 169.1 85.5909) (width 0.508) (layer "F.Cu") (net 2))
 (segment (start 144.175 92.24) (end 144.175 93.8) (width 0.508) (layer "F.Cu") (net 2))
 (segment (start 169.1 85.5909) (end 169.1 85.5) (width 0.508) (layer "F.Cu") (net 2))
 (segment (start 144.175 87.16) (end 144.175 85.6) (width 0.508) (layer "F.Cu") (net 2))
 (segment (start 147.375 92) (end 147.375 93.1) (width 0.508) (layer "F.Cu") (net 2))
 (segment (start 162.275 85.6) (end 162.275 86.575) (width 0.508) (layer "F.Cu") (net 2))
 (via (at 144.175 85.6) (size 0.6) (drill 0.3) (layers "F.Cu" "B.Cu") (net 2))
 (via (at 156.7 90.9) (size 0.6) (drill 0.3) (layers "F.Cu" "B.Cu") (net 2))
 (via (at 162.3 86.6) (size 0.6) (drill 0.3) (layers "F.Cu" "B.Cu") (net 2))
 (via (at 156.7 86.7) (size 0.6) (drill 0.3) (layers "F.Cu" "B.Cu") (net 2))
 (via (at 165.9 93) (size 0.6) (drill 0.3) (layers "F.Cu" "B.Cu") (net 2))
 (via (at 144.175 93.8) (size 0.6) (drill 0.3) (layers "F.Cu" "B.Cu") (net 2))
 (via (at 169.1 85.5) (size 0.6) (drill 0.3) (layers "F.Cu" "B.Cu") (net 2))
 (via (at 169 93.8) (size 0.6) (drill 0.3) (layers "F.Cu" "B.Cu") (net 2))
 (via (at 169.8 83.4) (size 0.6) (drill 0.3) (layers "F.Cu" "B.Cu") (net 2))
 (via (at 147.375 93.1) (size 0.6) (drill 0.3) (layers "F.Cu" "B.Cu") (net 2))
 (segment (start 149.2 87.7) (end 149.2 84.96) (width 0.508) (layer "F.Cu") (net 7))
 (segment (start 149.2 84.96) (end 150.56 83.6) (width 0.508) (layer "F.Cu") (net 7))
 (segment (start 144.175 89.7) (end 149.1 89.7) (width 1.2019) (layer "F.Cu") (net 1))
 (segment (start 164.1375 89.7) (end 169.04545 89.7) (width 1.2019) (layer "F.Cu") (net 6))
 (segment (start 160.2 89.7) (end 158.6 89.7) (width 1.2019) (layer "F.Cu") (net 9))
 (segment (start 160.2 89.7) (end 162.0625 89.7) (width 1.2019) (layer "F.Cu") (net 9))
 (segment (start 164.6 83.4) (end 166.5 83.4) (width 0.508) (layer "F.Cu") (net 5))
 (segment (start 164.6 83.4) (end 164.6 81.2) (width 0.508) (layer "F.Cu") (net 5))
 (segment (start 164.6 81.2) (end 163.8 80.4) (width 0.508) (layer "F.Cu") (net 5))
 (segment (start 160.2 83.4) (end 160.2 87.4) (width 0.508) (layer "F.Cu") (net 3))
 (segment (start 160 83.6) (end 160.2 83.4) (width 0.508) (layer "F.Cu") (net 3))
 (segment (start 153.1 87.7) (end 153.1 83.6) (width 0.508) (layer "F.Cu") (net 3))
 (segment (start 153.1 83.6) (end 160 83.6) (width 0.508) (layer "F.Cu") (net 3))
 (segment (start 153.1 89.7) (end 154.8 89.7) (width 1.2019) (layer "F.Cu") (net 4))
 (segment (start 151.175 89.7) (end 153.1 89.7) (width 1.2019) (layer "F.Cu") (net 4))
 (segment (start 151.175 87.725) (end 151.2 87.7) (width 1.2019) (layer "F.Cu") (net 8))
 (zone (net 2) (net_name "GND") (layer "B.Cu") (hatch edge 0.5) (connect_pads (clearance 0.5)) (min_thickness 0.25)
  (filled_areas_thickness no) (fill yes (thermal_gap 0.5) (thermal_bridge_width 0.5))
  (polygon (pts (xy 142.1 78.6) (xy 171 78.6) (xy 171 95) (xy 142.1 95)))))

